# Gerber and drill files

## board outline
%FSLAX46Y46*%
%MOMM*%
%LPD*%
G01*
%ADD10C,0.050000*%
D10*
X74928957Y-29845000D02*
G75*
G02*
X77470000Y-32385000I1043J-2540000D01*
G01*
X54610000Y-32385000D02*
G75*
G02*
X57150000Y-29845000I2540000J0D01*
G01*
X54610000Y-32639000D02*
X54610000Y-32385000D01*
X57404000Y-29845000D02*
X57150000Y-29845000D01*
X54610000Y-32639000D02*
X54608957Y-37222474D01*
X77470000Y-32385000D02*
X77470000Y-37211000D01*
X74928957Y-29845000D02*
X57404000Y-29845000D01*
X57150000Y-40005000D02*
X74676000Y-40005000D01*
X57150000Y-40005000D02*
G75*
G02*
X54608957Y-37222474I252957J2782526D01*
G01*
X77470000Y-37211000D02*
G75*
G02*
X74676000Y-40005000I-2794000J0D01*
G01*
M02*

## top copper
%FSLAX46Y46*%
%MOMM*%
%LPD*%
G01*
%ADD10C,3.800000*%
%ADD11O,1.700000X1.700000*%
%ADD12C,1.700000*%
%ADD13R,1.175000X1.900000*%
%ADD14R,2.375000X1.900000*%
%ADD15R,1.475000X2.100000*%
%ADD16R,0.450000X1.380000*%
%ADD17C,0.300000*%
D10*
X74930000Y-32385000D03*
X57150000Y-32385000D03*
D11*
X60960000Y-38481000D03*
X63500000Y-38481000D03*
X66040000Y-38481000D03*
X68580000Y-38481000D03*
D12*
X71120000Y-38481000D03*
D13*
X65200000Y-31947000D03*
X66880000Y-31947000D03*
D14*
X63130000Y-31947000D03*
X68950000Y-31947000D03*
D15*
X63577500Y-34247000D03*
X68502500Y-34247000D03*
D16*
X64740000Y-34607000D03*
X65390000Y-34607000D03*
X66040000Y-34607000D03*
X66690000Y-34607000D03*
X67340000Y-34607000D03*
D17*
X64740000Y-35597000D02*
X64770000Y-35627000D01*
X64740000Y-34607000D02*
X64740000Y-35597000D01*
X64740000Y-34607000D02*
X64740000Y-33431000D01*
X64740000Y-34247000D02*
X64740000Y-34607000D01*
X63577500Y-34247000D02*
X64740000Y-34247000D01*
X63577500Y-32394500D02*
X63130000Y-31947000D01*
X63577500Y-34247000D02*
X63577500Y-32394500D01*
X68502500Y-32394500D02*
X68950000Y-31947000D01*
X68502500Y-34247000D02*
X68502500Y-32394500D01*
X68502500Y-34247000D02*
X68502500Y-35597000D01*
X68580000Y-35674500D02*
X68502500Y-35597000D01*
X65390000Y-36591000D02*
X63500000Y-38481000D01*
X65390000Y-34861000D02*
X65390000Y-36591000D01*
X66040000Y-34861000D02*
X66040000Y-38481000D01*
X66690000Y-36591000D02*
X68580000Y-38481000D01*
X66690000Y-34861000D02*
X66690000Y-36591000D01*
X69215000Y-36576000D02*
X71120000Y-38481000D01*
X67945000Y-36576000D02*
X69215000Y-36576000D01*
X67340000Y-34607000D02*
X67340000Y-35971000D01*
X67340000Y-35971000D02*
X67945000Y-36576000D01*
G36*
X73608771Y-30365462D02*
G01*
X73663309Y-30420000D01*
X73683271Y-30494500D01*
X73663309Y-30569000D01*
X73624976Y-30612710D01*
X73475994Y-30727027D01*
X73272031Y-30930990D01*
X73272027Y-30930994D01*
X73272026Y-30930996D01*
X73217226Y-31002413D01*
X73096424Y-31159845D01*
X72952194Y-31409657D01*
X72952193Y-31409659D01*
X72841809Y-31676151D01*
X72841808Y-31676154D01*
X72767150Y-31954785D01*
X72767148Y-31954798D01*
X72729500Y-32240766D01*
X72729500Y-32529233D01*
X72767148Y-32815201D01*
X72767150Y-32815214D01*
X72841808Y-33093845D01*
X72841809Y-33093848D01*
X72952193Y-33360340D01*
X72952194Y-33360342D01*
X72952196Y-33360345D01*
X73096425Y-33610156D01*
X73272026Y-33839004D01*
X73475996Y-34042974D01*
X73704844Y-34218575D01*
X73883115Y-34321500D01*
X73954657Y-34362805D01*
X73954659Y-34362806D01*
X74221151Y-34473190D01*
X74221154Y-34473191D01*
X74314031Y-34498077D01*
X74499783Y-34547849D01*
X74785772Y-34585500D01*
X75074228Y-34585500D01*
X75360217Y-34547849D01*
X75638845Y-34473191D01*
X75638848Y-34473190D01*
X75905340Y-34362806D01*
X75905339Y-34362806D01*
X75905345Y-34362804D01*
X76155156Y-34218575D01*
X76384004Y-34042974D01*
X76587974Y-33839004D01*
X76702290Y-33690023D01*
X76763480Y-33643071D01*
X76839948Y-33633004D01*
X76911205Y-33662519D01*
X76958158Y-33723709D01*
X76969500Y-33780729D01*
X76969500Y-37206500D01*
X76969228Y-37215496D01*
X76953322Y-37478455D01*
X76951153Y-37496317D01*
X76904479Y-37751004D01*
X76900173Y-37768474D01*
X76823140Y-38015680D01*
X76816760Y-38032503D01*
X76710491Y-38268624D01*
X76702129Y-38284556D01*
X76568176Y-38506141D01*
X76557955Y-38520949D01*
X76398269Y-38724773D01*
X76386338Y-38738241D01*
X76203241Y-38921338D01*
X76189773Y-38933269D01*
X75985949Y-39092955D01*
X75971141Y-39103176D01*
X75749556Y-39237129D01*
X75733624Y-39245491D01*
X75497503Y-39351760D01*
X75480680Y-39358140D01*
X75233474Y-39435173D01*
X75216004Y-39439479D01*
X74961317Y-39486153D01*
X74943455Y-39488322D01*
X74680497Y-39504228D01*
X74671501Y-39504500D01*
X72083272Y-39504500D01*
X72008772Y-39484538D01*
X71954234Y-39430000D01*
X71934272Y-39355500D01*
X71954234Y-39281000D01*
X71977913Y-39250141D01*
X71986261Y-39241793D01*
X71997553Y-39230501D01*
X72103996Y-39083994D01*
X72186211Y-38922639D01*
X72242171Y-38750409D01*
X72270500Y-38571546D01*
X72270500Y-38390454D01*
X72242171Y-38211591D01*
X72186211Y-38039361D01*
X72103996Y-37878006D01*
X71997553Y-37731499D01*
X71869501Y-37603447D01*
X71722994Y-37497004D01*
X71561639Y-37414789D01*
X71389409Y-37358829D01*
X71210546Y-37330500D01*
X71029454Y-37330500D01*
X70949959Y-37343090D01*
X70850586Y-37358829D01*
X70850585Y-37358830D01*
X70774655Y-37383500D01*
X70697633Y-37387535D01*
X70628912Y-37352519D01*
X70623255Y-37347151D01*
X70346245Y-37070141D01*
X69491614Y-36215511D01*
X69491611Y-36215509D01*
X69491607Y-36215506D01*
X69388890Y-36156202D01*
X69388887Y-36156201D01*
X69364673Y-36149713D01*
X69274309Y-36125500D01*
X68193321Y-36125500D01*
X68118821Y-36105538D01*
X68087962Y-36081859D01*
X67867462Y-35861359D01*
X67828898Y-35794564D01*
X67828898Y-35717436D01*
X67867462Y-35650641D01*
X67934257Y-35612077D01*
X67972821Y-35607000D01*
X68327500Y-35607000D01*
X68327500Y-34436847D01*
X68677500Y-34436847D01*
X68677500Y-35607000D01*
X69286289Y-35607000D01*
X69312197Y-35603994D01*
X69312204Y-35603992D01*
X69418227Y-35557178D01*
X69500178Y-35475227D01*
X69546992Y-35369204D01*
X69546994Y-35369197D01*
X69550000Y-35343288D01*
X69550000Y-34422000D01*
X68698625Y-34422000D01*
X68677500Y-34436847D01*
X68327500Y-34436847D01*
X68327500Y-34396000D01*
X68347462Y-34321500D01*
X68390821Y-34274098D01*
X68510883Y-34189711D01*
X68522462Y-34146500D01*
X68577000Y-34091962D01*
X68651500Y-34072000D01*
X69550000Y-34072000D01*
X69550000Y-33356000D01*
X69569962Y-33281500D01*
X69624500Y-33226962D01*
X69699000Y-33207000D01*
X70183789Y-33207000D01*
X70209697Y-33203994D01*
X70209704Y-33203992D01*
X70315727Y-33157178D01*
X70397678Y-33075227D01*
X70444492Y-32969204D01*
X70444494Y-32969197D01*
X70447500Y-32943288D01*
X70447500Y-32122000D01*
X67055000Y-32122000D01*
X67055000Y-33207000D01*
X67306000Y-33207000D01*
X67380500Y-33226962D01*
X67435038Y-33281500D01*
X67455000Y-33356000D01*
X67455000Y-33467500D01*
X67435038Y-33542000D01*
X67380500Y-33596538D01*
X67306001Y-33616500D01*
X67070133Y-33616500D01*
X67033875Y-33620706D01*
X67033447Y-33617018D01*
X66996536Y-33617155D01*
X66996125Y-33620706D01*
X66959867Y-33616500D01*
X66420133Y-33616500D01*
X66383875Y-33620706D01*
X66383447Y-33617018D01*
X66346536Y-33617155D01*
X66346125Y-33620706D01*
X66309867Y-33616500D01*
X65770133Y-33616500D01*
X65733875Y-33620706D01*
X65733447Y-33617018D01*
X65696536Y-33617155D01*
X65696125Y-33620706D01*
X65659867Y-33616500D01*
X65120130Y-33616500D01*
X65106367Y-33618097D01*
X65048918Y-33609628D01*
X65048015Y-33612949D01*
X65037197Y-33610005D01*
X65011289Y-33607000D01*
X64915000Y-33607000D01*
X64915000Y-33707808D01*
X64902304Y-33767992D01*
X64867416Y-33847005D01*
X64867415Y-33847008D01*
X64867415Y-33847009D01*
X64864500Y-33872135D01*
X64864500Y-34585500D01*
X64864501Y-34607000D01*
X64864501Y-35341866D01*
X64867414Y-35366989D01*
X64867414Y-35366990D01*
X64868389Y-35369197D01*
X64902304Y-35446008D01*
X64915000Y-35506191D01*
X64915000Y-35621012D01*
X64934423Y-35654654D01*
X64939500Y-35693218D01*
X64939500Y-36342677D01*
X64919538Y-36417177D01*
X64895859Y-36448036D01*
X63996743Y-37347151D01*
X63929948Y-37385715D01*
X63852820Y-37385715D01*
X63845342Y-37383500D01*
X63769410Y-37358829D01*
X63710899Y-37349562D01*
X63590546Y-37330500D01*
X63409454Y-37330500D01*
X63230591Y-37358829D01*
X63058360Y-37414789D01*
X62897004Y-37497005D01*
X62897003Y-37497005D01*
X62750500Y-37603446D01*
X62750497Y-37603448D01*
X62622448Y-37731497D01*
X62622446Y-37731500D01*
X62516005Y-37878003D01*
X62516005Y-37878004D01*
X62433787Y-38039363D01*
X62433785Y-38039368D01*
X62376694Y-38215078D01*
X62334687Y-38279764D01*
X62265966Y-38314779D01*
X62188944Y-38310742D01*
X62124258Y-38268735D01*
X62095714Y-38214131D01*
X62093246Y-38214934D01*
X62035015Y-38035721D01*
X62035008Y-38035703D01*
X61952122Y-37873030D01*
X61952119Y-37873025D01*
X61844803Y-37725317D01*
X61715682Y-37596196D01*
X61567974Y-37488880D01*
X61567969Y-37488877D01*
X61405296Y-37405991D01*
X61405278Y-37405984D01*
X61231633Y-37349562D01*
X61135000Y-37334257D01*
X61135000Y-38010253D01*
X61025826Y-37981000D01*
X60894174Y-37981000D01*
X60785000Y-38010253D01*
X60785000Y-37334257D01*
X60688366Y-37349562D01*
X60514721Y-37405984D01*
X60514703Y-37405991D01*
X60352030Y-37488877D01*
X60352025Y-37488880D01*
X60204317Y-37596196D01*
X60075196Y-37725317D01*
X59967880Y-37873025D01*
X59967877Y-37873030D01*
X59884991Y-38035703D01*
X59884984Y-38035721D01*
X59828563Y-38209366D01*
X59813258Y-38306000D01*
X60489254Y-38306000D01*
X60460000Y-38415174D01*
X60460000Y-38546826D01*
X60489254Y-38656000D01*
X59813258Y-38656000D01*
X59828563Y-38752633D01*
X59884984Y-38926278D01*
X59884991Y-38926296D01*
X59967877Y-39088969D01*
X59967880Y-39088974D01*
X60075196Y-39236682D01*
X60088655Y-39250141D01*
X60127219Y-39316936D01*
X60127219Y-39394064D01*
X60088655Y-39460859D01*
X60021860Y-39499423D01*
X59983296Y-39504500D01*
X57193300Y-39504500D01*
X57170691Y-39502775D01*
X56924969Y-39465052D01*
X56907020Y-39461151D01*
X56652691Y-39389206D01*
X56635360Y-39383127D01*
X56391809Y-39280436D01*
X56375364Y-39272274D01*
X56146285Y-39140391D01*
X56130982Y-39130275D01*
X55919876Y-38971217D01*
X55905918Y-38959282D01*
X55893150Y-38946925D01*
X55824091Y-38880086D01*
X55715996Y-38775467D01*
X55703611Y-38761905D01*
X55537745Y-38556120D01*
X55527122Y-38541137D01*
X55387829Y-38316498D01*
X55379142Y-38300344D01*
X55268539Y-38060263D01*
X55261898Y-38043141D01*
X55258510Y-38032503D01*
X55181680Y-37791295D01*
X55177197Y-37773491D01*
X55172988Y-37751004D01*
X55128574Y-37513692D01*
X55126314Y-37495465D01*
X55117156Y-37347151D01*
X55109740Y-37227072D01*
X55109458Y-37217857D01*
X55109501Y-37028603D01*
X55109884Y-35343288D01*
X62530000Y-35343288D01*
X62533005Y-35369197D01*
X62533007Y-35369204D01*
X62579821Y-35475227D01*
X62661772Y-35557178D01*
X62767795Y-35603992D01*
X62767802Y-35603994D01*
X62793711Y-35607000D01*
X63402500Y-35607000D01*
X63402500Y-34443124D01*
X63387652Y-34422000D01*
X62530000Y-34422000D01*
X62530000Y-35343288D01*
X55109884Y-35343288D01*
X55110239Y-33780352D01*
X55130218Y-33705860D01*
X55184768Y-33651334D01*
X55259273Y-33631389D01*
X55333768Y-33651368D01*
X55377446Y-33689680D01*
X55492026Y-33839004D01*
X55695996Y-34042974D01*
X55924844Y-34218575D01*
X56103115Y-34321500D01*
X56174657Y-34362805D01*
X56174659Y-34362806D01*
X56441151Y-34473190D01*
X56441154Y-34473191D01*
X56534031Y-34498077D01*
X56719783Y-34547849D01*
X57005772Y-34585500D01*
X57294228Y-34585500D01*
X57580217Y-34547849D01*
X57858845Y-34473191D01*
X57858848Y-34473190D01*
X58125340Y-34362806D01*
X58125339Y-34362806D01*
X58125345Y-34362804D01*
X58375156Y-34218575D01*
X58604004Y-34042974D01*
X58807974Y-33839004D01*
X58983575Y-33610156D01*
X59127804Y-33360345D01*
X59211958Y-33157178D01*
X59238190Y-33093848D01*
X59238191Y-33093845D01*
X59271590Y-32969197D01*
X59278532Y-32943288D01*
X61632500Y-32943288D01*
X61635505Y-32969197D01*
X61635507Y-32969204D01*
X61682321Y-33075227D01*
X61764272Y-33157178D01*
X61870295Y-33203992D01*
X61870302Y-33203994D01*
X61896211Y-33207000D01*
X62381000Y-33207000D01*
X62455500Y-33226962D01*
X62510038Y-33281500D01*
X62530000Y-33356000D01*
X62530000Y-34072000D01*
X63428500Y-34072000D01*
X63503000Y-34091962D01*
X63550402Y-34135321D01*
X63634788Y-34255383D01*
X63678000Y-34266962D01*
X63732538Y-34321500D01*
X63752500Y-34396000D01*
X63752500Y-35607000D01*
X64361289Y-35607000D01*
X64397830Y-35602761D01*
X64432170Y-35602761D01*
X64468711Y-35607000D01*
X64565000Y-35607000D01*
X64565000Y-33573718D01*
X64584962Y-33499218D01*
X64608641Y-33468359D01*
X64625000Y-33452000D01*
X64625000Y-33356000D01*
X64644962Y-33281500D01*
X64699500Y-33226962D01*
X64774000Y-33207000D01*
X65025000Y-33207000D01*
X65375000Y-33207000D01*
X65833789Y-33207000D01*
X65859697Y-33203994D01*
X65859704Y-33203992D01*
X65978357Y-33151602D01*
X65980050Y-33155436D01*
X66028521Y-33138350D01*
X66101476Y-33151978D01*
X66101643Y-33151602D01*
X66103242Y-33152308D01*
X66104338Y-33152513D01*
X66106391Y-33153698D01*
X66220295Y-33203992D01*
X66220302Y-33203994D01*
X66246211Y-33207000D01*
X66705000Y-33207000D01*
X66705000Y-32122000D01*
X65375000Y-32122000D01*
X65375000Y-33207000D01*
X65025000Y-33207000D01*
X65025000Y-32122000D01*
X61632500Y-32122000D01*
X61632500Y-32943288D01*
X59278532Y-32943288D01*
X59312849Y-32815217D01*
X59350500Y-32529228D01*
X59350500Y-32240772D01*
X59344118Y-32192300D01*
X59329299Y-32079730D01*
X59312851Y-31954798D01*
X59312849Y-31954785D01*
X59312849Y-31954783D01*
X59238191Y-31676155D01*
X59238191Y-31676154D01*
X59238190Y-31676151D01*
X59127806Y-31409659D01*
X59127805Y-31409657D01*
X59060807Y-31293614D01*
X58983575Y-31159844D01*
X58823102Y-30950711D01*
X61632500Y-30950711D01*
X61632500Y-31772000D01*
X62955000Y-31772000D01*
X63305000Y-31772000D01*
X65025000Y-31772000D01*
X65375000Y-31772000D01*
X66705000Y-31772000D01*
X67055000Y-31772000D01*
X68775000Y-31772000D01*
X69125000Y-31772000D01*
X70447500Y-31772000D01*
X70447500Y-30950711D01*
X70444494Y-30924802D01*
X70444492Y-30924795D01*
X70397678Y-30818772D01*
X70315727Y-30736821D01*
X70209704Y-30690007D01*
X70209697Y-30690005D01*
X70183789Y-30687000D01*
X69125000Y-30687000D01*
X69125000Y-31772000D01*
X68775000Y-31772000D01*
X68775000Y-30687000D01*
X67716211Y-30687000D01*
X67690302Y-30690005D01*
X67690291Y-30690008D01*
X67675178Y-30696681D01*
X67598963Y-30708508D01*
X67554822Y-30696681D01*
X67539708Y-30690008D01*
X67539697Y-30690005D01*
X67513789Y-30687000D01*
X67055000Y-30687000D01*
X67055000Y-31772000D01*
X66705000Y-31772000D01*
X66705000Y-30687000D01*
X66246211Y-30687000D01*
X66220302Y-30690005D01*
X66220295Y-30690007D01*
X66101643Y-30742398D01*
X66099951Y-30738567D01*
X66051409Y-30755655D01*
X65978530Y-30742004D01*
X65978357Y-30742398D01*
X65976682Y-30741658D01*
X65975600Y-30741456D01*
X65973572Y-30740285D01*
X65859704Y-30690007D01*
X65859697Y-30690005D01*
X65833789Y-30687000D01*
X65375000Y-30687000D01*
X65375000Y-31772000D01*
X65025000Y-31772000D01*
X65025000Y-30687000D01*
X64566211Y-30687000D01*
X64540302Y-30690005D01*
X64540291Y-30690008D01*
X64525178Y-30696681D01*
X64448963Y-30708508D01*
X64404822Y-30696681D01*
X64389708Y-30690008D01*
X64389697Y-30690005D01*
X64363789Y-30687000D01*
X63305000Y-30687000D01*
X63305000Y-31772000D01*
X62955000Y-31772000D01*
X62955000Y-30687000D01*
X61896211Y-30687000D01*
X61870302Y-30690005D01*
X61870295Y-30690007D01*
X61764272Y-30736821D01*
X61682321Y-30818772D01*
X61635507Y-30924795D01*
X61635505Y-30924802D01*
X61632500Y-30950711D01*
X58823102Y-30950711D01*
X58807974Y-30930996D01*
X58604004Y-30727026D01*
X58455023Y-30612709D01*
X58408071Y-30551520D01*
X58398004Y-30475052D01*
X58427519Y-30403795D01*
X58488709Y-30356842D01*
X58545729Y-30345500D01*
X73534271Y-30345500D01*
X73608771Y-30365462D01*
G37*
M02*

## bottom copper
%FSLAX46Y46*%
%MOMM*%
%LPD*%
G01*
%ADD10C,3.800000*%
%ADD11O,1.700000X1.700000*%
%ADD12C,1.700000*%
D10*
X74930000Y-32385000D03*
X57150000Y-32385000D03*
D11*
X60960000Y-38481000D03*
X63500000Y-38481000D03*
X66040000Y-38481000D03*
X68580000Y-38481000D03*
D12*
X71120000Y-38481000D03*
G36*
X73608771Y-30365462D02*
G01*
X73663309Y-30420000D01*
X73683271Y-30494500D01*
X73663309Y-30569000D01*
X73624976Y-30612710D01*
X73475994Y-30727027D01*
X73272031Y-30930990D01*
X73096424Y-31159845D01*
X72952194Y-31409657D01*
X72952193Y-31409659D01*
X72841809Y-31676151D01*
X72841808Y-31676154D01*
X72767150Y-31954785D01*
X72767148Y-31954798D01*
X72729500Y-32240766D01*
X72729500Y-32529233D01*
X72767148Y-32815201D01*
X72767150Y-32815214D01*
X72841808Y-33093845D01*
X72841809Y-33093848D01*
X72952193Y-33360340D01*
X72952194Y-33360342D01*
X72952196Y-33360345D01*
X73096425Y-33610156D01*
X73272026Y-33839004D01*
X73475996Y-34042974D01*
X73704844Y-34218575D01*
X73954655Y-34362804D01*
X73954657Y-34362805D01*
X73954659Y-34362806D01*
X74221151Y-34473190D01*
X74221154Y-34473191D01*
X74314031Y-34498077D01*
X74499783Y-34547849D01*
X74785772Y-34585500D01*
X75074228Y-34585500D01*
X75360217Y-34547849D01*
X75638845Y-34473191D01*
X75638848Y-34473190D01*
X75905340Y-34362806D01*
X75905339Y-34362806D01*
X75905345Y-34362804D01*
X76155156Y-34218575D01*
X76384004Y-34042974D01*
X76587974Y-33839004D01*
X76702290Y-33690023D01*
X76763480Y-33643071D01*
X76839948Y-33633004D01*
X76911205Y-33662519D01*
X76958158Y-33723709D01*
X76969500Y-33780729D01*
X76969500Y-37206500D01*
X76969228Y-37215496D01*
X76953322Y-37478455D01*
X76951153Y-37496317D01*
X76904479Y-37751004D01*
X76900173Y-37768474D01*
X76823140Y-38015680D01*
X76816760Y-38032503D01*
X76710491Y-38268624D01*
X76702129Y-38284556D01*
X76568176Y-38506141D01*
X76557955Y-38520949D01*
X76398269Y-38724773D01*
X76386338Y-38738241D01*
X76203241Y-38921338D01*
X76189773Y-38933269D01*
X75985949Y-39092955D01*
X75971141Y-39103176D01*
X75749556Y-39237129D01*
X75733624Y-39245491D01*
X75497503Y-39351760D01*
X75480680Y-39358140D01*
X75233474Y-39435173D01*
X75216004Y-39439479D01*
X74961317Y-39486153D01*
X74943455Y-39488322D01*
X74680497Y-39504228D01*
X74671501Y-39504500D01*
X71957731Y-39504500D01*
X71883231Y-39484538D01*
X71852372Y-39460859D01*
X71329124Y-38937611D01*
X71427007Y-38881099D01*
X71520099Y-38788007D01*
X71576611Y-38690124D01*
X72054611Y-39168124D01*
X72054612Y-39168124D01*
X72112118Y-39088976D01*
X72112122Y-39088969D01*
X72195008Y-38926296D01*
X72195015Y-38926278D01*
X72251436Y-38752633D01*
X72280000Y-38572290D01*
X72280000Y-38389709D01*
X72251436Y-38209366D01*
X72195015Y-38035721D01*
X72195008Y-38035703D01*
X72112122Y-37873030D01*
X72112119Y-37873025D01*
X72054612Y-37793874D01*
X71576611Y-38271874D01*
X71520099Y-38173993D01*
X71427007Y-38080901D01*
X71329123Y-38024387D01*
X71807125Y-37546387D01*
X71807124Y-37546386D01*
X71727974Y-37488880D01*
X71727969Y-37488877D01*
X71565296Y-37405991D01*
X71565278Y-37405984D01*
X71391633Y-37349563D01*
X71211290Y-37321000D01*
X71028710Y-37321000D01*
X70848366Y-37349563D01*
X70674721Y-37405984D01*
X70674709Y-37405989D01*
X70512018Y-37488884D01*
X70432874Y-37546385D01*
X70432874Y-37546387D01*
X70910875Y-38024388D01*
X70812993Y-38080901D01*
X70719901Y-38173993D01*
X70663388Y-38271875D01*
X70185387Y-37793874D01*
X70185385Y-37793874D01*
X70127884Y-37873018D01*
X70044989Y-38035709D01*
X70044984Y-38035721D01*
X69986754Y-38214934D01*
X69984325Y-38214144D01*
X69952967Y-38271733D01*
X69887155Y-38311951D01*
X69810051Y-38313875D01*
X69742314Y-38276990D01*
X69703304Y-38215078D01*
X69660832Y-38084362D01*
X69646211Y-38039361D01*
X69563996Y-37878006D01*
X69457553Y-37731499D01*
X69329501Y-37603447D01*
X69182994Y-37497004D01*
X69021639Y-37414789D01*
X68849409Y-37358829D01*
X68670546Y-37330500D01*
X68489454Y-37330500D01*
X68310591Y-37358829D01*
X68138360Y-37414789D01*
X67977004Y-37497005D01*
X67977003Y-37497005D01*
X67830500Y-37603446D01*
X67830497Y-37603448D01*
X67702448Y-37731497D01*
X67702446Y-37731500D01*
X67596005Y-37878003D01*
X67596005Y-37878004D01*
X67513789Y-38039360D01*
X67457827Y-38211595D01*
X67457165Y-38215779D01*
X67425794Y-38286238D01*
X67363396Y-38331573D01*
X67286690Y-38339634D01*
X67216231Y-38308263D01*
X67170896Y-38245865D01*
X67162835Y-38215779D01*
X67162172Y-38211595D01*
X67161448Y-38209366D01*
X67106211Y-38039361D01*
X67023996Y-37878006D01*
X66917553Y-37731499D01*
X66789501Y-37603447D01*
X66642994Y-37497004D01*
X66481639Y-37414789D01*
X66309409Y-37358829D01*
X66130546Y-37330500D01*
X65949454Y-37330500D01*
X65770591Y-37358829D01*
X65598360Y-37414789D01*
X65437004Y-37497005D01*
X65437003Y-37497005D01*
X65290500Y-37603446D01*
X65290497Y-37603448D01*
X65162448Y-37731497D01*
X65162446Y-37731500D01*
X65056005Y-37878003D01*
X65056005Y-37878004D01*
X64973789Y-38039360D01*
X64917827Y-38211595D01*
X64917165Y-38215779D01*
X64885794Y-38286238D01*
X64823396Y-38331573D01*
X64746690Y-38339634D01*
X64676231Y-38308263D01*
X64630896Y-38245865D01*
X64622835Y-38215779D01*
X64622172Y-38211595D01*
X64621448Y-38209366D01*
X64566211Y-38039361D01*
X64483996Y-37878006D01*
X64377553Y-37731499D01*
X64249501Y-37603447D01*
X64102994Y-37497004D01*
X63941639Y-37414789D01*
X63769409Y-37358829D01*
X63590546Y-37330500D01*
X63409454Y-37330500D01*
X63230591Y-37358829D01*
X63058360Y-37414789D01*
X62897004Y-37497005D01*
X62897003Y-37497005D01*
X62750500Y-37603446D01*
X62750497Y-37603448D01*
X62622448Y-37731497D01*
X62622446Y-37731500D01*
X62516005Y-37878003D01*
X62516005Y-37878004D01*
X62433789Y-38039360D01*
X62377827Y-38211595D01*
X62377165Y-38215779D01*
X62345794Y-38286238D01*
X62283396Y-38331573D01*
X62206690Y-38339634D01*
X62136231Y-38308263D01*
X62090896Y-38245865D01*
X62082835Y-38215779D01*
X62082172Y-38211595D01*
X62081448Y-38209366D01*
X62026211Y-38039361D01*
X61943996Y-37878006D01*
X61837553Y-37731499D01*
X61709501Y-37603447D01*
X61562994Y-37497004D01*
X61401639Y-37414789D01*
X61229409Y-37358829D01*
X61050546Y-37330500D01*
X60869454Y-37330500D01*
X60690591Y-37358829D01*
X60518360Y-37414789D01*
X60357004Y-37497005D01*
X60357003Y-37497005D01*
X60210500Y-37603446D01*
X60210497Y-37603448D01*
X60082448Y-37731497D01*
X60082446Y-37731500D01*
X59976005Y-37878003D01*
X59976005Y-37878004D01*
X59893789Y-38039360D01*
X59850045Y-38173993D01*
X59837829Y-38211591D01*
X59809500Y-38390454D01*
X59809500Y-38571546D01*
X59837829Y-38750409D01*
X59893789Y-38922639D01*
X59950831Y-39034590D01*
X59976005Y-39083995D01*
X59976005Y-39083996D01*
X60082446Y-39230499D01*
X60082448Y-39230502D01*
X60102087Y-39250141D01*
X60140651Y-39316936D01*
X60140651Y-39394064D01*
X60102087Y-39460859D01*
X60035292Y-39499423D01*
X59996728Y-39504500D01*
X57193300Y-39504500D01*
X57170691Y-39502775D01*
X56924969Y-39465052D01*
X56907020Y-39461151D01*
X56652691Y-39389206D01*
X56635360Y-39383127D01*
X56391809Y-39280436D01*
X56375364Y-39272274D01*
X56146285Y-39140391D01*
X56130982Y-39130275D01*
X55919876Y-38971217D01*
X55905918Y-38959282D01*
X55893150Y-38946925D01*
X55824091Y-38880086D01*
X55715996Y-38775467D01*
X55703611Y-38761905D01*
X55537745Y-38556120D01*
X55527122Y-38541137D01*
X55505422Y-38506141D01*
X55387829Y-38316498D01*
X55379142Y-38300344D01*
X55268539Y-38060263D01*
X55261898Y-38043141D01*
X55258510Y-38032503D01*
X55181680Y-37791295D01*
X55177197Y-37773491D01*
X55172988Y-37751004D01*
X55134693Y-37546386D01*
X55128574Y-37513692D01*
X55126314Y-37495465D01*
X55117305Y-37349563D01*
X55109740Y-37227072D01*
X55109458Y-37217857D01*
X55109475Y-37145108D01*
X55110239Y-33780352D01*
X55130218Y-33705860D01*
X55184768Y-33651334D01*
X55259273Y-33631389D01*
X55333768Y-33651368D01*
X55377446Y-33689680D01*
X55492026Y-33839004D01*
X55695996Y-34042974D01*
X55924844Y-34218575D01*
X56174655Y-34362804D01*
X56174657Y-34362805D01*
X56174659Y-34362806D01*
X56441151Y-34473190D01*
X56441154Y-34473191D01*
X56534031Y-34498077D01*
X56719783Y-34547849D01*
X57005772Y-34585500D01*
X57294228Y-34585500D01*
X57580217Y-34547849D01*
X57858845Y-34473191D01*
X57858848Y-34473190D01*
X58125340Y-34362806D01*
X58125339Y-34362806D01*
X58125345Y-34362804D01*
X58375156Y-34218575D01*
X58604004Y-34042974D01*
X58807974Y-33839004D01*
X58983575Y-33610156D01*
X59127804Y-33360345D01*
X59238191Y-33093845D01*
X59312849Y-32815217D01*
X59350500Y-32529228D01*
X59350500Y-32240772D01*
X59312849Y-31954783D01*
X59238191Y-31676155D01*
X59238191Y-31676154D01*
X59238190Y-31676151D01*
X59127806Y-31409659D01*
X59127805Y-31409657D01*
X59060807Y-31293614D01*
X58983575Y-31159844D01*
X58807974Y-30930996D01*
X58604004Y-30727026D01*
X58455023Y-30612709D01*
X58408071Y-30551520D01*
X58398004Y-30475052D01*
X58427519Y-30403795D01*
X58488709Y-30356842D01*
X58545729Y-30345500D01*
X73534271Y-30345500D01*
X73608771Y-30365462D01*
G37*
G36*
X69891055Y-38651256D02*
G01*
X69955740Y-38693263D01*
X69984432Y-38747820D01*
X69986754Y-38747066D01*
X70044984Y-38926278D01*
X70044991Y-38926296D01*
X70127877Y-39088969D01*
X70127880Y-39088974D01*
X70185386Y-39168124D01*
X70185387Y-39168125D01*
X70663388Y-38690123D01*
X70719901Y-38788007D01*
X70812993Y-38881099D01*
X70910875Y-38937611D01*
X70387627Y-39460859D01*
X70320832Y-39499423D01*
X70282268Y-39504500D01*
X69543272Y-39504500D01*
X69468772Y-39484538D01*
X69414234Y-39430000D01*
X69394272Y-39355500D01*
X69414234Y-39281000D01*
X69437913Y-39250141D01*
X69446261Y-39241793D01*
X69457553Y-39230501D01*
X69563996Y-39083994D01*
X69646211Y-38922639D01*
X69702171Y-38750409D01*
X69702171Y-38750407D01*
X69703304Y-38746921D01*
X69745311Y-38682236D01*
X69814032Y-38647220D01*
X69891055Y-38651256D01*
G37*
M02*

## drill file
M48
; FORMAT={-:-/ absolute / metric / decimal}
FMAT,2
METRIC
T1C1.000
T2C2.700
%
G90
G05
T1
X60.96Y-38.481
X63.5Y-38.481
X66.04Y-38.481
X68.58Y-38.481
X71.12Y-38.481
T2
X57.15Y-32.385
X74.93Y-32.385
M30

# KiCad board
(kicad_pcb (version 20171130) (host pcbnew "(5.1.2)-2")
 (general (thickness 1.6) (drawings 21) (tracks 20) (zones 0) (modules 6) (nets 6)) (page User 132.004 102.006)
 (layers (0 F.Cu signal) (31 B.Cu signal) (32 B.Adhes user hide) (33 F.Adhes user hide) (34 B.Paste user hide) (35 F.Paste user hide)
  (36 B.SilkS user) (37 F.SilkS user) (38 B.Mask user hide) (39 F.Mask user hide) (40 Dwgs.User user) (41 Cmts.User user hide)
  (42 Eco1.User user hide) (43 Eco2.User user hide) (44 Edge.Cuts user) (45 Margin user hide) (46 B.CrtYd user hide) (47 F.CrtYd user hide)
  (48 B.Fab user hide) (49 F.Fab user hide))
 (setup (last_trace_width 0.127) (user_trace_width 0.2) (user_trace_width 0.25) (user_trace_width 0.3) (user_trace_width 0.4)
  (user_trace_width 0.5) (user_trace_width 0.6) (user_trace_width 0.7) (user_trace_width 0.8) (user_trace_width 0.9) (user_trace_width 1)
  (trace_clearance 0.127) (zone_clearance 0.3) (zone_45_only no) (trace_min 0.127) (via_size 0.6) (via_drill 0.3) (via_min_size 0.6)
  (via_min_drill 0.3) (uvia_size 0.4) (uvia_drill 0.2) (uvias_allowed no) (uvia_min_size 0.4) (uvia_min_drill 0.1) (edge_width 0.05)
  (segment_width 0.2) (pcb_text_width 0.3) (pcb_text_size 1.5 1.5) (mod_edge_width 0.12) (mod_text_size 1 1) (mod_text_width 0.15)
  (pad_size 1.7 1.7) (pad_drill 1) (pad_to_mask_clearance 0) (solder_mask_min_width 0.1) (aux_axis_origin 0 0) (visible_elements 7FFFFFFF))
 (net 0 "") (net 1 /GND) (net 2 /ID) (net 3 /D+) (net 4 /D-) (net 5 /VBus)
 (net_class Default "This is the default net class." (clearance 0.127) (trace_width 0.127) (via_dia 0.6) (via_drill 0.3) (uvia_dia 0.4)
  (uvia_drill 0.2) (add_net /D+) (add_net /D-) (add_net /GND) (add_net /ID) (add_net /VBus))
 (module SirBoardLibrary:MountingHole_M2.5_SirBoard (layer F.Cu) (at 74.93 32.385)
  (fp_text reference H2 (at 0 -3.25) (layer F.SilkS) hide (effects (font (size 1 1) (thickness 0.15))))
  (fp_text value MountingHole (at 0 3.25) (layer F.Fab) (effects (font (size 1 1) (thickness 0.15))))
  (pad 1 thru_hole circle (at 0 0) (size 3.8 3.8) (drill 2.7) (layers *.Cu *.Mask)))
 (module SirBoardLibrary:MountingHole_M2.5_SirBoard (layer F.Cu) (at 57.15 32.385)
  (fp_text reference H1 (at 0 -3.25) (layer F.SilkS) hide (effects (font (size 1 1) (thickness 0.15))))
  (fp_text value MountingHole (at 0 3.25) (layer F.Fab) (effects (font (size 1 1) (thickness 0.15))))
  (pad 1 thru_hole circle (at 0 0) (size 3.8 3.8) (drill 2.7) (layers *.Cu *.Mask)))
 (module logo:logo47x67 (layer B.Cu) (at 66.04 32.639 180)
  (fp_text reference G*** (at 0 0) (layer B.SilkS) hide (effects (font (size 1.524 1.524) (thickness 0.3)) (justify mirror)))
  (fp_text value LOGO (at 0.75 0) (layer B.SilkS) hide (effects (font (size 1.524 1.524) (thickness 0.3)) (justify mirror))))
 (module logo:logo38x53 (layer F.Cu) (at 57.404 36.957)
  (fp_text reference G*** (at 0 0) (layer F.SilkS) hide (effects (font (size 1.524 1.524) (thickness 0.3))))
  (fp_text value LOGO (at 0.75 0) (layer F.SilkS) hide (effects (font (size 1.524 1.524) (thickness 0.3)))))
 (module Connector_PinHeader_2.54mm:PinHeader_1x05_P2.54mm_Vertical (layer B.Cu) (at 71.12 38.481 90)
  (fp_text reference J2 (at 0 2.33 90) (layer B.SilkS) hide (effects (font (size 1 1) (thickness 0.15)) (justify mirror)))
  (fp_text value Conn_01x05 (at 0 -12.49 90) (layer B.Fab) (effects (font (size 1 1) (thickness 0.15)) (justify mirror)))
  (pad 5 thru_hole oval (at 0 -10.16 90) (size 1.7 1.7) (drill 1) (layers *.Cu *.Mask) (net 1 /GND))
  (pad 4 thru_hole oval (at 0 -7.62 90) (size 1.7 1.7) (drill 1) (layers *.Cu *.Mask) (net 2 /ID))
  (pad 3 thru_hole oval (at 0 -5.08 90) (size 1.7 1.7) (drill 1) (layers *.Cu *.Mask) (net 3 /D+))
  (pad 2 thru_hole oval (at 0 -2.54 90) (size 1.7 1.7) (drill 1) (layers *.Cu *.Mask) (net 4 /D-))
  (pad 1 thru_hole circle (at 0 0 90) (size 1.7 1.7) (drill 1) (layers *.Cu *.Mask) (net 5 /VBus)))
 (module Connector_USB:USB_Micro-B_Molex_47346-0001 (layer F.Cu) (at 66.04 33.147 180)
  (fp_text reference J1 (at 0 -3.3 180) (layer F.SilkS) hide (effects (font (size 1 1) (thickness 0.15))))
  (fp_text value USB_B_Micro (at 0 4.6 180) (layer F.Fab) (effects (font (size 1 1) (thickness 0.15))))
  (pad 6 smd rect (at 0.84 1.2 180) (size 1.175 1.9) (layers F.Cu F.Paste F.Mask) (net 1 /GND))
  (pad 6 smd rect (at -0.84 1.2 180) (size 1.175 1.9) (layers F.Cu F.Paste F.Mask) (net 1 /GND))
  (pad 6 smd rect (at 2.91 1.2 180) (size 2.375 1.9) (layers F.Cu F.Paste F.Mask) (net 1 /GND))
  (pad 6 smd rect (at -2.91 1.2 180) (size 2.375 1.9) (layers F.Cu F.Paste F.Mask) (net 1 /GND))
  (pad 6 smd rect (at 2.4625 -1.1 180) (size 1.475 2.1) (layers F.Cu F.Paste F.Mask) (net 1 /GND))
  (pad 6 smd rect (at -2.4625 -1.1 180) (size 1.475 2.1) (layers F.Cu F.Paste F.Mask) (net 1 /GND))
  (pad 5 smd rect (at 1.3 -1.46 180) (size 0.45 1.38) (layers F.Cu F.Paste F.Mask) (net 1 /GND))
  (pad 4 smd rect (at 0.65 -1.46 180) (size 0.45 1.38) (layers F.Cu F.Paste F.Mask) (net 2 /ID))
  (pad 3 smd rect (at 0 -1.46 180) (size 0.45 1.38) (layers F.Cu F.Paste F.Mask) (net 3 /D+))
  (pad 2 smd rect (at -0.65 -1.46 180) (size 0.45 1.38) (layers F.Cu F.Paste F.Mask) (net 4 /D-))
  (pad 1 smd rect (at -1.3 -1.46 180) (size 0.45 1.38) (layers F.Cu F.Paste F.Mask) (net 5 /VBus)))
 (gr_arc (start 74.93 32.385) (end 77.47 32.385) (angle -90.02352736) (layer Edge.Cuts) (width 0.05))
 (gr_arc (start 57.15 32.385) (end 57.15 29.845) (angle -90) (layer Edge.Cuts) (width 0.05))
 (gr_line (start 54.61 32.639) (end 54.61 32.385) (layer Edge.Cuts) (width 0.05))
 (gr_line (start 57.404 29.845) (end 57.15 29.845) (layer Edge.Cuts) (width 0.05))
 (gr_line (start 54.61 32.639) (end 54.608957 37.222474) (layer Edge.Cuts) (width 0.05))
 (gr_line (start 77.47 32.385) (end 77.47 37.211) (layer Edge.Cuts) (width 0.05))
 (gr_line (start 74.928957 29.845) (end 57.404 29.845) (layer Edge.Cuts) (width 0.05))
 (gr_line (start 57.15 40.005) (end 74.676 40.005) (layer Edge.Cuts) (width 0.05))
 (gr_arc (start 57.402957 37.222474) (end 54.608957 37.222474) (angle -84.80557109) (layer Edge.Cuts) (width 0.05))
 (gr_arc (start 74.676 37.211) (end 74.676 40.005) (angle -90) (layer Edge.Cuts) (width 0.05))
 (segment (start 64.74 35.597) (end 64.77 35.627) (width 0.3) (layer F.Cu) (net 1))
 (segment (start 64.74 34.607) (end 64.74 35.597) (width 0.3) (layer F.Cu) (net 1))
 (segment (start 64.74 34.607) (end 64.74 33.431) (width 0.3) (layer F.Cu) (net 1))
 (segment (start 64.74 34.247) (end 64.74 34.607) (width 0.3) (layer F.Cu) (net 1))
 (segment (start 63.5775 34.247) (end 64.74 34.247) (width 0.3) (layer F.Cu) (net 1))
 (segment (start 63.5775 32.3945) (end 63.13 31.947) (width 0.3) (layer F.Cu) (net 1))
 (segment (start 63.5775 34.247) (end 63.5775 32.3945) (width 0.3) (layer F.Cu) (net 1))
 (segment (start 68.5025 32.3945) (end 68.95 31.947) (width 0.3) (layer F.Cu) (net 1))
 (segment (start 68.5025 34.247) (end 68.5025 32.3945) (width 0.3) (layer F.Cu) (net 1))
 (segment (start 68.5025 34.247) (end 68.5025 35.597) (width 0.3) (layer F.Cu) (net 1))
 (segment (start 68.58 35.6745) (end 68.5025 35.597) (width 0.3) (layer F.Cu) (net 1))
 (segment (start 65.39 36.591) (end 63.5 38.481) (width 0.3) (layer F.Cu) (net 2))
 (segment (start 65.39 34.861) (end 65.39 36.591) (width 0.3) (layer F.Cu) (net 2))
 (segment (start 66.04 34.861) (end 66.04 38.481) (width 0.3) (layer F.Cu) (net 3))
 (segment (start 66.69 36.591) (end 68.58 38.481) (width 0.3) (layer F.Cu) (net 4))
 (segment (start 66.69 34.861) (end 66.69 36.591) (width 0.3) (layer F.Cu) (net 4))
 (segment (start 69.215 36.576) (end 71.12 38.481) (width 0.3) (layer F.Cu) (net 5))
 (segment (start 67.945 36.576) (end 69.215 36.576) (width 0.3) (layer F.Cu) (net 5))
 (segment (start 67.34 34.607) (end 67.34 35.971) (width 0.3) (layer F.Cu) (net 5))
 (segment (start 67.34 35.971) (end 67.945 36.576) (width 0.3) (layer F.Cu) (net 5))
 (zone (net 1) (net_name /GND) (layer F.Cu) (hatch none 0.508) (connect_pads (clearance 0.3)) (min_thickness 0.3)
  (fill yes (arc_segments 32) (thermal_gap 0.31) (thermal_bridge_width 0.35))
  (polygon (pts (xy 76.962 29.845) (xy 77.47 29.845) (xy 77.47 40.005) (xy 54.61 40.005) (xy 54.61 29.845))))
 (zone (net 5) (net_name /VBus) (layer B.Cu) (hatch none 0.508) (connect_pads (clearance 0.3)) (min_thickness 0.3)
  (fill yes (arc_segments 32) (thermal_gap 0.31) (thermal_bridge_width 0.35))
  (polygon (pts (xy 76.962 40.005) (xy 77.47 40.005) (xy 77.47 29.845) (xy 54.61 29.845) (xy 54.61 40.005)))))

